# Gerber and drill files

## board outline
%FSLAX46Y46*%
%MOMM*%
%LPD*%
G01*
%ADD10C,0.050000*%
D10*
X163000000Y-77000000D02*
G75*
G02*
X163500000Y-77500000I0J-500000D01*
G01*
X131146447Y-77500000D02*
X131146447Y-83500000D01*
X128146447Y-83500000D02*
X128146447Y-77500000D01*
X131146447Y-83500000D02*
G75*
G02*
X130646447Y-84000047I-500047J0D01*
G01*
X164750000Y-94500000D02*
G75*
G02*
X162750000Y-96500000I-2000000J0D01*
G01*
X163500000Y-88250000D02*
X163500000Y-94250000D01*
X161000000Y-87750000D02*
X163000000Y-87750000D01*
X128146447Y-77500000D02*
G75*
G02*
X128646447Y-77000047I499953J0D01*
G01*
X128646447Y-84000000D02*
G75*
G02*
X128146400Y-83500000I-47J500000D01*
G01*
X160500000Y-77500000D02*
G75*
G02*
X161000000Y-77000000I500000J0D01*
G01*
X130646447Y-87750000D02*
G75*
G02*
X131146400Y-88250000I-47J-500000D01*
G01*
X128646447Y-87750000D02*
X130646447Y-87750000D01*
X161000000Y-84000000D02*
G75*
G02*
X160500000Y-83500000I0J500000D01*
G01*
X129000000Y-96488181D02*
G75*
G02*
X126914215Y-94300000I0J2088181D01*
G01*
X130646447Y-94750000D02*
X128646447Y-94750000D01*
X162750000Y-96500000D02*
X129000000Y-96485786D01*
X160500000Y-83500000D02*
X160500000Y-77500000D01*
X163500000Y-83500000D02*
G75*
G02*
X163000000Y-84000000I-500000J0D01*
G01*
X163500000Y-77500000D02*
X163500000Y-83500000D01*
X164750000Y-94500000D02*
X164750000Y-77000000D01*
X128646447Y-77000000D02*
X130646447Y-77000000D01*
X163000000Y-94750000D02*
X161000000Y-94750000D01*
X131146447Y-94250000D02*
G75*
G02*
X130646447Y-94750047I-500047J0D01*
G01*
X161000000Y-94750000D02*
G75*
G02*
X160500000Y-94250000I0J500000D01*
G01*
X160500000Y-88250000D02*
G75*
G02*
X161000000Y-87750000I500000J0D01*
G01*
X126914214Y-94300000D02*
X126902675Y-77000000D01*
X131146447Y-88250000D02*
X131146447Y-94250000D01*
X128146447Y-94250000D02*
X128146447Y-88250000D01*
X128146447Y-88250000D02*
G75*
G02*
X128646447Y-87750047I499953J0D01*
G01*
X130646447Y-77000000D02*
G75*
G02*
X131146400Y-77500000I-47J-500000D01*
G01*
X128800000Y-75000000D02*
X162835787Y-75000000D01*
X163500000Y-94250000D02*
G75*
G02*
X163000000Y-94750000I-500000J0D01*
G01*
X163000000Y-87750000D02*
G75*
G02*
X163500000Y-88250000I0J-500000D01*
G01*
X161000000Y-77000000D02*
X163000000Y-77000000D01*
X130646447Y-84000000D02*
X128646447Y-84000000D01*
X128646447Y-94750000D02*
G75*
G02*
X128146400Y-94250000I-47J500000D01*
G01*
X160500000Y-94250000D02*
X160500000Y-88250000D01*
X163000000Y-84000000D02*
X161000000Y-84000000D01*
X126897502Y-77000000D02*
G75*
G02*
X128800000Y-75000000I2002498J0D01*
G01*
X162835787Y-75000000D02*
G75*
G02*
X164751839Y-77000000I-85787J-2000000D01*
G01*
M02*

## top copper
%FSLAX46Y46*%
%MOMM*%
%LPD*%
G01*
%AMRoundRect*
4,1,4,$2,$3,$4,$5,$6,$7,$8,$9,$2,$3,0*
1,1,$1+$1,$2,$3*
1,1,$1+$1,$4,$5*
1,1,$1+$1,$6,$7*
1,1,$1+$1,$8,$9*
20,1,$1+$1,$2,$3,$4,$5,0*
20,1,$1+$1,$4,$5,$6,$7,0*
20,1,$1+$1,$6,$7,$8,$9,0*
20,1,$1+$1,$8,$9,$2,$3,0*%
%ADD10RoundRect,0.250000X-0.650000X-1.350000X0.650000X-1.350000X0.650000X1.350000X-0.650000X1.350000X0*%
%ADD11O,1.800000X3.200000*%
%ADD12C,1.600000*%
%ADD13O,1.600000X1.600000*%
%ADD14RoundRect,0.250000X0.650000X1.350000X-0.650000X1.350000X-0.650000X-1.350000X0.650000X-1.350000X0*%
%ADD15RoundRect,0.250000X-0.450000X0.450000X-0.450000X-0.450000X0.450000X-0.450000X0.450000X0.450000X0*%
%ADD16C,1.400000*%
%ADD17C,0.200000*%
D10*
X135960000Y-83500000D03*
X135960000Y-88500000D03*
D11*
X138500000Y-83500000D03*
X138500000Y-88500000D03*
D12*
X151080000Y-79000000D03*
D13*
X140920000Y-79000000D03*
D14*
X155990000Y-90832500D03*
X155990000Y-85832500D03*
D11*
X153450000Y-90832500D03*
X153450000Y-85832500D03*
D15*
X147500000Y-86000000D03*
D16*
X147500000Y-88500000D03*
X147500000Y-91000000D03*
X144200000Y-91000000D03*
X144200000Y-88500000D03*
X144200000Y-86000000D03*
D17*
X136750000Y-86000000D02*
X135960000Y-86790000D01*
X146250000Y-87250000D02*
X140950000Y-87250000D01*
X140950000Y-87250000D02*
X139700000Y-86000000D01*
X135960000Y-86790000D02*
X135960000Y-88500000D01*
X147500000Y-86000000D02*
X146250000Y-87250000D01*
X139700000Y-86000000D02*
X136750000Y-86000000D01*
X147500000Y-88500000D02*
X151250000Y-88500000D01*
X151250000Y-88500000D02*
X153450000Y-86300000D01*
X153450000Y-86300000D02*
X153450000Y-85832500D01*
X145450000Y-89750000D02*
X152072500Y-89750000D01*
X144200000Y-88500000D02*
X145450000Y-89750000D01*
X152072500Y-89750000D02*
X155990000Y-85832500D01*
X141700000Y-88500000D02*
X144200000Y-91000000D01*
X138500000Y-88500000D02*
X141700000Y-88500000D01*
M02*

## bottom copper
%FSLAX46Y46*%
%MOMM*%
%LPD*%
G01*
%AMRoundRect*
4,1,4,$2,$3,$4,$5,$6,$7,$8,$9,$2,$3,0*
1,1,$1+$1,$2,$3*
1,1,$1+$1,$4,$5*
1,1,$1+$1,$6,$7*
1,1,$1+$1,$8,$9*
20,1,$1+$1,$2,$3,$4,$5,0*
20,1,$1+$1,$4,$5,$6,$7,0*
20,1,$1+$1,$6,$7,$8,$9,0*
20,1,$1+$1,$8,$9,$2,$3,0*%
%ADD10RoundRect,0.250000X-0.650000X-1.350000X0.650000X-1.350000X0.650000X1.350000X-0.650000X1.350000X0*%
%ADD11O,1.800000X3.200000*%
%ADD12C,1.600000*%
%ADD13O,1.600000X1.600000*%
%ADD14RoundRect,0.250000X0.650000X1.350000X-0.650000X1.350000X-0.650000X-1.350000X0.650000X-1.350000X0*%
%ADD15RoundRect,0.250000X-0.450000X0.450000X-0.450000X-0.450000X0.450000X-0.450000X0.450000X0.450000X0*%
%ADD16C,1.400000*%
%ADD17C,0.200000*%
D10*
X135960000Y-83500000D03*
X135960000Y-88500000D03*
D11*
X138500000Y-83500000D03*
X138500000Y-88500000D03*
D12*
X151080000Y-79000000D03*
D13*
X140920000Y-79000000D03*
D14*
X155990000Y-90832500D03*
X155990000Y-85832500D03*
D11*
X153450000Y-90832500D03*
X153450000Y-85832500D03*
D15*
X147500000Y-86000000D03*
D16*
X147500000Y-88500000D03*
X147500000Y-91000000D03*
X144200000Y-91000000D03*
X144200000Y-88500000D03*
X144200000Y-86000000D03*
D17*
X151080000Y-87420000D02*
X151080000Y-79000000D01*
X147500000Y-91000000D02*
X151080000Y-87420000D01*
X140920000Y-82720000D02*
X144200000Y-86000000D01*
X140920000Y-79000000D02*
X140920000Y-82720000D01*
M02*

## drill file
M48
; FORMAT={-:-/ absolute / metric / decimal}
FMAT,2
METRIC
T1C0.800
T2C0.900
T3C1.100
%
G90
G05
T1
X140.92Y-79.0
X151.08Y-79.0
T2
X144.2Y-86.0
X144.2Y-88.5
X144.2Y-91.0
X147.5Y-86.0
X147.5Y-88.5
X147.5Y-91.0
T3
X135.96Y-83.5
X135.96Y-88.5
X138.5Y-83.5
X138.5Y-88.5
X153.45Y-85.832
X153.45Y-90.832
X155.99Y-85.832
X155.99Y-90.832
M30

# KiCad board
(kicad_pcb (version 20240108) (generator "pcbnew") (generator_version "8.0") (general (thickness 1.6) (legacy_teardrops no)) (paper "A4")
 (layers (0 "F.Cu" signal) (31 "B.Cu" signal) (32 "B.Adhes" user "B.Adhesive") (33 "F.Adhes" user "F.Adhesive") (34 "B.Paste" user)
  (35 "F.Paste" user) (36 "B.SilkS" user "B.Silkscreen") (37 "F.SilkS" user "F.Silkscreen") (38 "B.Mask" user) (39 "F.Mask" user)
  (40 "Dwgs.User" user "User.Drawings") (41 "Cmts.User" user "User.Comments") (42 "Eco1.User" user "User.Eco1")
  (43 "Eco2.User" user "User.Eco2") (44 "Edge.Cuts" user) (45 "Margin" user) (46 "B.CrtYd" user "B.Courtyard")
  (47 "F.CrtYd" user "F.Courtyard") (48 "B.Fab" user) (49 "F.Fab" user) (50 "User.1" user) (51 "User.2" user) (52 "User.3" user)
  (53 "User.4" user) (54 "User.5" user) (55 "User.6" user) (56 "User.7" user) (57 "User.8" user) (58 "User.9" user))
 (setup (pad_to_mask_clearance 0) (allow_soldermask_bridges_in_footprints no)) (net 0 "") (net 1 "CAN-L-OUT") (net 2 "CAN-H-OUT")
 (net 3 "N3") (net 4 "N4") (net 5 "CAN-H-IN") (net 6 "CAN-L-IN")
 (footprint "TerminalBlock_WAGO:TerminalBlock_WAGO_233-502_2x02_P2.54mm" (layer "F.Cu") (at 135.96 83.5)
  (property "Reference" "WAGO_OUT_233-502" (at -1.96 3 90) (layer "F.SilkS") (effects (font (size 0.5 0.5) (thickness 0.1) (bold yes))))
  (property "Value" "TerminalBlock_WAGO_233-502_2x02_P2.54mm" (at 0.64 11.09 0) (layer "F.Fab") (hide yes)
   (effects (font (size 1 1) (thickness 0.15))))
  (pad "1" thru_hole roundrect (at 0 0) (size 1.8 3.2) (drill 1.1) (layers "*.Cu" "*.Mask") (remove_unused_layers no)
   (roundrect_rratio 0.1388888889))
  (pad "1" thru_hole roundrect (at 0 5) (size 1.8 3.2) (drill 1.1) (layers "*.Cu" "*.Mask") (remove_unused_layers no)
   (roundrect_rratio 0.1388888889) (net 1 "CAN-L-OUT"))
  (pad "2" thru_hole oval (at 2.54 0) (size 1.8 3.2) (drill 1.1) (layers "*.Cu" "*.Mask") (remove_unused_layers no))
  (pad "2" thru_hole oval (at 2.54 5) (size 1.8 3.2) (drill 1.1) (layers "*.Cu" "*.Mask") (remove_unused_layers no) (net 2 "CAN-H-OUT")))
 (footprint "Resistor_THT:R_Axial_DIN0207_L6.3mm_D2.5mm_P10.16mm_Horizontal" (layer "F.Cu") (at 151.08 79 180)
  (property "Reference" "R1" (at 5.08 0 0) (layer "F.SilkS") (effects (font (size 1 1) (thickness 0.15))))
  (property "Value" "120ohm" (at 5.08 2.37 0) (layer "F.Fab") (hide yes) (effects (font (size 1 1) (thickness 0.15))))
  (pad "1" thru_hole circle (at 0 0 180) (size 1.6 1.6) (drill 0.8) (layers "*.Cu" "*.Mask") (remove_unused_layers no) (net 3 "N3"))
  (pad "2" thru_hole oval (at 10.16 0 180) (size 1.6 1.6) (drill 0.8) (layers "*.Cu" "*.Mask") (remove_unused_layers no) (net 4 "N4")))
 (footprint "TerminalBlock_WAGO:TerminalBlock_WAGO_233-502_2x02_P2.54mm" (layer "F.Cu") (at 155.99 90.8325 180)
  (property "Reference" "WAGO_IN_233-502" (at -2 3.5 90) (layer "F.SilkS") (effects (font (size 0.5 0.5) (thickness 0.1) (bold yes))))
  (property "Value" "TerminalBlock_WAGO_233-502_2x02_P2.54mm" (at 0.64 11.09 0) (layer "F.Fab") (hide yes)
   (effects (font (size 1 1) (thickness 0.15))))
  (pad "1" thru_hole roundrect (at 0 0 180) (size 1.8 3.2) (drill 1.1) (layers "*.Cu" "*.Mask") (remove_unused_layers no)
   (roundrect_rratio 0.1388888889))
  (pad "1" thru_hole roundrect (at 0 5 180) (size 1.8 3.2) (drill 1.1) (layers "*.Cu" "*.Mask") (remove_unused_layers no)
   (roundrect_rratio 0.1388888889) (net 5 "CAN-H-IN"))
  (pad "2" thru_hole oval (at 2.54 0 180) (size 1.8 3.2) (drill 1.1) (layers "*.Cu" "*.Mask") (remove_unused_layers no))
  (pad "2" thru_hole oval (at 2.54 5 180) (size 1.8 3.2) (drill 1.1) (layers "*.Cu" "*.Mask") (remove_unused_layers no) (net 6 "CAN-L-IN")))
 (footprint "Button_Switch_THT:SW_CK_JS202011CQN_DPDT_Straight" (layer "F.Cu") (at 147.5 86 -90)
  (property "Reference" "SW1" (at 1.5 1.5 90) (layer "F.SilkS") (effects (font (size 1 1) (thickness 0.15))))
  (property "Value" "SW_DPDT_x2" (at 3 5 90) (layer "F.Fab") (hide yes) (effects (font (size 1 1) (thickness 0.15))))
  (pad "1" thru_hole roundrect (at 0 0 270) (size 1.4 1.4) (drill 0.9) (layers "*.Cu" "*.Mask") (remove_unused_layers no)
   (roundrect_rratio 0.1785714286) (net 1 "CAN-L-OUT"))
  (pad "2" thru_hole circle (at 2.5 0 270) (size 1.4 1.4) (drill 0.9) (layers "*.Cu" "*.Mask") (remove_unused_layers no) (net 6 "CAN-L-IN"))
  (pad "3" thru_hole circle (at 5 0 270) (size 1.4 1.4) (drill 0.9) (layers "*.Cu" "*.Mask") (remove_unused_layers no) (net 3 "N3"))
  (pad "4" thru_hole circle (at 5 3.3 270) (size 1.4 1.4) (drill 0.9) (layers "*.Cu" "*.Mask") (remove_unused_layers no) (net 2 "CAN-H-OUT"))
  (pad "5" thru_hole circle (at 2.5 3.3 270) (size 1.4 1.4) (drill 0.9) (layers "*.Cu" "*.Mask") (remove_unused_layers no)
   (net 5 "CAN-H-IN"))
  (pad "6" thru_hole circle (at 0 3.3 270) (size 1.4 1.4) (drill 0.9) (layers "*.Cu" "*.Mask") (remove_unused_layers no) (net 4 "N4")))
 (gr_arc (start 163 77) (mid 163.353553 77.146447) (end 163.5 77.5) (stroke (width 0.05) (type default)) (layer "Edge.Cuts"))
 (gr_line (start 131.146447 77.5) (end 131.146447 83.5) (stroke (width 0.05) (type default)) (layer "Edge.Cuts"))
 (gr_line (start 128.146447 83.5) (end 128.146447 77.5) (stroke (width 0.05) (type default)) (layer "Edge.Cuts"))
 (gr_arc (start 131.146447 83.5) (mid 131 83.853553) (end 130.646447 84) (stroke (width 0.05) (type default)) (layer "Edge.Cuts"))
 (gr_arc (start 164.75 94.5) (mid 164.164213 95.914209) (end 162.75 96.5) (stroke (width 0.05) (type default)) (layer "Edge.Cuts"))
 (gr_line (start 163.5 88.25) (end 163.5 94.25) (stroke (width 0.05) (type default)) (layer "Edge.Cuts"))
 (gr_line (start 161 87.75) (end 163 87.75) (stroke (width 0.05) (type default)) (layer "Edge.Cuts"))
 (gr_arc (start 128.146447 77.5) (mid 128.292894 77.146447) (end 128.646447 77) (stroke (width 0.05) (type default)) (layer "Edge.Cuts"))
 (gr_arc (start 128.646447 84) (mid 128.292894 83.853553) (end 128.146447 83.5) (stroke (width 0.05) (type default)) (layer "Edge.Cuts"))
 (gr_arc (start 160.5 77.5) (mid 160.646447 77.146447) (end 161 77) (stroke (width 0.05) (type default)) (layer "Edge.Cuts"))
 (gr_arc (start 130.646447 87.75) (mid 131 87.896447) (end 131.146447 88.25) (stroke (width 0.05) (type default)) (layer "Edge.Cuts"))
 (gr_line (start 128.646447 87.75) (end 130.646447 87.75) (stroke (width 0.05) (type default)) (layer "Edge.Cuts"))
 (gr_arc (start 161 84) (mid 160.646447 83.853553) (end 160.5 83.5) (stroke (width 0.05) (type default)) (layer "Edge.Cuts"))
 (gr_arc (start 129 96.488181) (mid 127.488491 95.840778) (end 126.914215 94.3) (stroke (width 0.05) (type default)) (layer "Edge.Cuts"))
 (gr_line (start 130.646447 94.75) (end 128.646447 94.75) (stroke (width 0.05) (type default)) (layer "Edge.Cuts"))
 (gr_line (start 162.75 96.5) (end 129 96.485786) (stroke (width 0.05) (type default)) (layer "Edge.Cuts"))
 (gr_line (start 160.5 83.5) (end 160.5 77.5) (stroke (width 0.05) (type default)) (layer "Edge.Cuts"))
 (gr_arc (start 163.5 83.5) (mid 163.353553 83.853553) (end 163 84) (stroke (width 0.05) (type default)) (layer "Edge.Cuts"))
 (gr_line (start 163.5 77.5) (end 163.5 83.5) (stroke (width 0.05) (type default)) (layer "Edge.Cuts"))
 (gr_line (start 164.75 94.5) (end 164.75 77) (stroke (width 0.05) (type default)) (layer "Edge.Cuts"))
 (gr_line (start 128.646447 77) (end 130.646447 77) (stroke (width 0.05) (type default)) (layer "Edge.Cuts"))
 (gr_line (start 163 94.75) (end 161 94.75) (stroke (width 0.05) (type default)) (layer "Edge.Cuts"))
 (gr_arc (start 131.146447 94.25) (mid 131 94.603553) (end 130.646447 94.75) (stroke (width 0.05) (type default)) (layer "Edge.Cuts"))
 (gr_arc (start 161 94.75) (mid 160.646447 94.603553) (end 160.5 94.25) (stroke (width 0.05) (type default)) (layer "Edge.Cuts"))
 (gr_arc (start 160.5 88.25) (mid 160.646447 87.896447) (end 161 87.75) (stroke (width 0.05) (type default)) (layer "Edge.Cuts"))
 (gr_line (start 126.914214 94.3) (end 126.902675 77) (stroke (width 0.05) (type default)) (layer "Edge.Cuts"))
 (gr_line (start 131.146447 88.25) (end 131.146447 94.25) (stroke (width 0.05) (type default)) (layer "Edge.Cuts"))
 (gr_line (start 128.146447 94.25) (end 128.146447 88.25) (stroke (width 0.05) (type default)) (layer "Edge.Cuts"))
 (gr_arc (start 128.146447 88.25) (mid 128.292894 87.896447) (end 128.646447 87.75) (stroke (width 0.05) (type default)) (layer "Edge.Cuts"))
 (gr_arc (start 130.646447 77) (mid 131 77.146447) (end 131.146447 77.5) (stroke (width 0.05) (type default)) (layer "Edge.Cuts"))
 (gr_line (start 128.8 75) (end 162.835787 75) (stroke (width 0.05) (type default)) (layer "Edge.Cuts"))
 (gr_arc (start 163.5 94.25) (mid 163.353553 94.603553) (end 163 94.75) (stroke (width 0.05) (type default)) (layer "Edge.Cuts"))
 (gr_arc (start 163 87.75) (mid 163.353553 87.896447) (end 163.5 88.25) (stroke (width 0.05) (type default)) (layer "Edge.Cuts"))
 (gr_line (start 161 77) (end 163 77) (stroke (width 0.05) (type default)) (layer "Edge.Cuts"))
 (gr_line (start 130.646447 84) (end 128.646447 84) (stroke (width 0.05) (type default)) (layer "Edge.Cuts"))
 (gr_arc (start 128.646447 94.75) (mid 128.292894 94.603553) (end 128.146447 94.25) (stroke (width 0.05) (type default)) (layer "Edge.Cuts"))
 (gr_line (start 160.5 94.25) (end 160.5 88.25) (stroke (width 0.05) (type default)) (layer "Edge.Cuts"))
 (gr_line (start 163 84) (end 161 84) (stroke (width 0.05) (type default)) (layer "Edge.Cuts"))
 (gr_arc (start 126.897502 77) (mid 127.449095 75.619828) (end 128.8 75) (stroke (width 0.05) (type default)) (layer "Edge.Cuts"))
 (gr_arc (start 162.835787 75) (mid 164.195526 75.615148) (end 164.751839 77) (stroke (width 0.05) (type default)) (layer "Edge.Cuts"))
 (segment (start 151.08 87.42) (end 151.08 79) (width 0.2) (layer "B.Cu") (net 3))
 (segment (start 147.5 91) (end 151.08 87.42) (width 0.2) (layer "B.Cu") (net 3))
 (segment (start 140.92 82.72) (end 144.2 86) (width 0.2) (layer "B.Cu") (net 4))
 (segment (start 140.92 79) (end 140.92 82.72) (width 0.2) (layer "B.Cu") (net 4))
 (segment (start 136.75 86) (end 135.96 86.79) (width 0.2) (layer "F.Cu") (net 1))
 (segment (start 146.25 87.25) (end 140.95 87.25) (width 0.2) (layer "F.Cu") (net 1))
 (segment (start 140.95 87.25) (end 139.7 86) (width 0.2) (layer "F.Cu") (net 1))
 (segment (start 135.96 86.79) (end 135.96 88.5) (width 0.2) (layer "F.Cu") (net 1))
 (segment (start 147.5 86) (end 146.25 87.25) (width 0.2) (layer "F.Cu") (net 1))
 (segment (start 139.7 86) (end 136.75 86) (width 0.2) (layer "F.Cu") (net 1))
 (segment (start 147.5 88.5) (end 151.25 88.5) (width 0.2) (layer "F.Cu") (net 6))
 (segment (start 151.25 88.5) (end 153.45 86.3) (width 0.2) (layer "F.Cu") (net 6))
 (segment (start 153.45 86.3) (end 153.45 85.8325) (width 0.2) (layer "F.Cu") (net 6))
 (segment (start 145.45 89.75) (end 152.0725 89.75) (width 0.2) (layer "F.Cu") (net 5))
 (segment (start 144.2 88.5) (end 145.45 89.75) (width 0.2) (layer "F.Cu") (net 5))
 (segment (start 152.0725 89.75) (end 155.99 85.8325) (width 0.2) (layer "F.Cu") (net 5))
 (segment (start 141.7 88.5) (end 144.2 91) (width 0.2) (layer "F.Cu") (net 2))
 (segment (start 138.5 88.5) (end 141.7 88.5) (width 0.2) (layer "F.Cu") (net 2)))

